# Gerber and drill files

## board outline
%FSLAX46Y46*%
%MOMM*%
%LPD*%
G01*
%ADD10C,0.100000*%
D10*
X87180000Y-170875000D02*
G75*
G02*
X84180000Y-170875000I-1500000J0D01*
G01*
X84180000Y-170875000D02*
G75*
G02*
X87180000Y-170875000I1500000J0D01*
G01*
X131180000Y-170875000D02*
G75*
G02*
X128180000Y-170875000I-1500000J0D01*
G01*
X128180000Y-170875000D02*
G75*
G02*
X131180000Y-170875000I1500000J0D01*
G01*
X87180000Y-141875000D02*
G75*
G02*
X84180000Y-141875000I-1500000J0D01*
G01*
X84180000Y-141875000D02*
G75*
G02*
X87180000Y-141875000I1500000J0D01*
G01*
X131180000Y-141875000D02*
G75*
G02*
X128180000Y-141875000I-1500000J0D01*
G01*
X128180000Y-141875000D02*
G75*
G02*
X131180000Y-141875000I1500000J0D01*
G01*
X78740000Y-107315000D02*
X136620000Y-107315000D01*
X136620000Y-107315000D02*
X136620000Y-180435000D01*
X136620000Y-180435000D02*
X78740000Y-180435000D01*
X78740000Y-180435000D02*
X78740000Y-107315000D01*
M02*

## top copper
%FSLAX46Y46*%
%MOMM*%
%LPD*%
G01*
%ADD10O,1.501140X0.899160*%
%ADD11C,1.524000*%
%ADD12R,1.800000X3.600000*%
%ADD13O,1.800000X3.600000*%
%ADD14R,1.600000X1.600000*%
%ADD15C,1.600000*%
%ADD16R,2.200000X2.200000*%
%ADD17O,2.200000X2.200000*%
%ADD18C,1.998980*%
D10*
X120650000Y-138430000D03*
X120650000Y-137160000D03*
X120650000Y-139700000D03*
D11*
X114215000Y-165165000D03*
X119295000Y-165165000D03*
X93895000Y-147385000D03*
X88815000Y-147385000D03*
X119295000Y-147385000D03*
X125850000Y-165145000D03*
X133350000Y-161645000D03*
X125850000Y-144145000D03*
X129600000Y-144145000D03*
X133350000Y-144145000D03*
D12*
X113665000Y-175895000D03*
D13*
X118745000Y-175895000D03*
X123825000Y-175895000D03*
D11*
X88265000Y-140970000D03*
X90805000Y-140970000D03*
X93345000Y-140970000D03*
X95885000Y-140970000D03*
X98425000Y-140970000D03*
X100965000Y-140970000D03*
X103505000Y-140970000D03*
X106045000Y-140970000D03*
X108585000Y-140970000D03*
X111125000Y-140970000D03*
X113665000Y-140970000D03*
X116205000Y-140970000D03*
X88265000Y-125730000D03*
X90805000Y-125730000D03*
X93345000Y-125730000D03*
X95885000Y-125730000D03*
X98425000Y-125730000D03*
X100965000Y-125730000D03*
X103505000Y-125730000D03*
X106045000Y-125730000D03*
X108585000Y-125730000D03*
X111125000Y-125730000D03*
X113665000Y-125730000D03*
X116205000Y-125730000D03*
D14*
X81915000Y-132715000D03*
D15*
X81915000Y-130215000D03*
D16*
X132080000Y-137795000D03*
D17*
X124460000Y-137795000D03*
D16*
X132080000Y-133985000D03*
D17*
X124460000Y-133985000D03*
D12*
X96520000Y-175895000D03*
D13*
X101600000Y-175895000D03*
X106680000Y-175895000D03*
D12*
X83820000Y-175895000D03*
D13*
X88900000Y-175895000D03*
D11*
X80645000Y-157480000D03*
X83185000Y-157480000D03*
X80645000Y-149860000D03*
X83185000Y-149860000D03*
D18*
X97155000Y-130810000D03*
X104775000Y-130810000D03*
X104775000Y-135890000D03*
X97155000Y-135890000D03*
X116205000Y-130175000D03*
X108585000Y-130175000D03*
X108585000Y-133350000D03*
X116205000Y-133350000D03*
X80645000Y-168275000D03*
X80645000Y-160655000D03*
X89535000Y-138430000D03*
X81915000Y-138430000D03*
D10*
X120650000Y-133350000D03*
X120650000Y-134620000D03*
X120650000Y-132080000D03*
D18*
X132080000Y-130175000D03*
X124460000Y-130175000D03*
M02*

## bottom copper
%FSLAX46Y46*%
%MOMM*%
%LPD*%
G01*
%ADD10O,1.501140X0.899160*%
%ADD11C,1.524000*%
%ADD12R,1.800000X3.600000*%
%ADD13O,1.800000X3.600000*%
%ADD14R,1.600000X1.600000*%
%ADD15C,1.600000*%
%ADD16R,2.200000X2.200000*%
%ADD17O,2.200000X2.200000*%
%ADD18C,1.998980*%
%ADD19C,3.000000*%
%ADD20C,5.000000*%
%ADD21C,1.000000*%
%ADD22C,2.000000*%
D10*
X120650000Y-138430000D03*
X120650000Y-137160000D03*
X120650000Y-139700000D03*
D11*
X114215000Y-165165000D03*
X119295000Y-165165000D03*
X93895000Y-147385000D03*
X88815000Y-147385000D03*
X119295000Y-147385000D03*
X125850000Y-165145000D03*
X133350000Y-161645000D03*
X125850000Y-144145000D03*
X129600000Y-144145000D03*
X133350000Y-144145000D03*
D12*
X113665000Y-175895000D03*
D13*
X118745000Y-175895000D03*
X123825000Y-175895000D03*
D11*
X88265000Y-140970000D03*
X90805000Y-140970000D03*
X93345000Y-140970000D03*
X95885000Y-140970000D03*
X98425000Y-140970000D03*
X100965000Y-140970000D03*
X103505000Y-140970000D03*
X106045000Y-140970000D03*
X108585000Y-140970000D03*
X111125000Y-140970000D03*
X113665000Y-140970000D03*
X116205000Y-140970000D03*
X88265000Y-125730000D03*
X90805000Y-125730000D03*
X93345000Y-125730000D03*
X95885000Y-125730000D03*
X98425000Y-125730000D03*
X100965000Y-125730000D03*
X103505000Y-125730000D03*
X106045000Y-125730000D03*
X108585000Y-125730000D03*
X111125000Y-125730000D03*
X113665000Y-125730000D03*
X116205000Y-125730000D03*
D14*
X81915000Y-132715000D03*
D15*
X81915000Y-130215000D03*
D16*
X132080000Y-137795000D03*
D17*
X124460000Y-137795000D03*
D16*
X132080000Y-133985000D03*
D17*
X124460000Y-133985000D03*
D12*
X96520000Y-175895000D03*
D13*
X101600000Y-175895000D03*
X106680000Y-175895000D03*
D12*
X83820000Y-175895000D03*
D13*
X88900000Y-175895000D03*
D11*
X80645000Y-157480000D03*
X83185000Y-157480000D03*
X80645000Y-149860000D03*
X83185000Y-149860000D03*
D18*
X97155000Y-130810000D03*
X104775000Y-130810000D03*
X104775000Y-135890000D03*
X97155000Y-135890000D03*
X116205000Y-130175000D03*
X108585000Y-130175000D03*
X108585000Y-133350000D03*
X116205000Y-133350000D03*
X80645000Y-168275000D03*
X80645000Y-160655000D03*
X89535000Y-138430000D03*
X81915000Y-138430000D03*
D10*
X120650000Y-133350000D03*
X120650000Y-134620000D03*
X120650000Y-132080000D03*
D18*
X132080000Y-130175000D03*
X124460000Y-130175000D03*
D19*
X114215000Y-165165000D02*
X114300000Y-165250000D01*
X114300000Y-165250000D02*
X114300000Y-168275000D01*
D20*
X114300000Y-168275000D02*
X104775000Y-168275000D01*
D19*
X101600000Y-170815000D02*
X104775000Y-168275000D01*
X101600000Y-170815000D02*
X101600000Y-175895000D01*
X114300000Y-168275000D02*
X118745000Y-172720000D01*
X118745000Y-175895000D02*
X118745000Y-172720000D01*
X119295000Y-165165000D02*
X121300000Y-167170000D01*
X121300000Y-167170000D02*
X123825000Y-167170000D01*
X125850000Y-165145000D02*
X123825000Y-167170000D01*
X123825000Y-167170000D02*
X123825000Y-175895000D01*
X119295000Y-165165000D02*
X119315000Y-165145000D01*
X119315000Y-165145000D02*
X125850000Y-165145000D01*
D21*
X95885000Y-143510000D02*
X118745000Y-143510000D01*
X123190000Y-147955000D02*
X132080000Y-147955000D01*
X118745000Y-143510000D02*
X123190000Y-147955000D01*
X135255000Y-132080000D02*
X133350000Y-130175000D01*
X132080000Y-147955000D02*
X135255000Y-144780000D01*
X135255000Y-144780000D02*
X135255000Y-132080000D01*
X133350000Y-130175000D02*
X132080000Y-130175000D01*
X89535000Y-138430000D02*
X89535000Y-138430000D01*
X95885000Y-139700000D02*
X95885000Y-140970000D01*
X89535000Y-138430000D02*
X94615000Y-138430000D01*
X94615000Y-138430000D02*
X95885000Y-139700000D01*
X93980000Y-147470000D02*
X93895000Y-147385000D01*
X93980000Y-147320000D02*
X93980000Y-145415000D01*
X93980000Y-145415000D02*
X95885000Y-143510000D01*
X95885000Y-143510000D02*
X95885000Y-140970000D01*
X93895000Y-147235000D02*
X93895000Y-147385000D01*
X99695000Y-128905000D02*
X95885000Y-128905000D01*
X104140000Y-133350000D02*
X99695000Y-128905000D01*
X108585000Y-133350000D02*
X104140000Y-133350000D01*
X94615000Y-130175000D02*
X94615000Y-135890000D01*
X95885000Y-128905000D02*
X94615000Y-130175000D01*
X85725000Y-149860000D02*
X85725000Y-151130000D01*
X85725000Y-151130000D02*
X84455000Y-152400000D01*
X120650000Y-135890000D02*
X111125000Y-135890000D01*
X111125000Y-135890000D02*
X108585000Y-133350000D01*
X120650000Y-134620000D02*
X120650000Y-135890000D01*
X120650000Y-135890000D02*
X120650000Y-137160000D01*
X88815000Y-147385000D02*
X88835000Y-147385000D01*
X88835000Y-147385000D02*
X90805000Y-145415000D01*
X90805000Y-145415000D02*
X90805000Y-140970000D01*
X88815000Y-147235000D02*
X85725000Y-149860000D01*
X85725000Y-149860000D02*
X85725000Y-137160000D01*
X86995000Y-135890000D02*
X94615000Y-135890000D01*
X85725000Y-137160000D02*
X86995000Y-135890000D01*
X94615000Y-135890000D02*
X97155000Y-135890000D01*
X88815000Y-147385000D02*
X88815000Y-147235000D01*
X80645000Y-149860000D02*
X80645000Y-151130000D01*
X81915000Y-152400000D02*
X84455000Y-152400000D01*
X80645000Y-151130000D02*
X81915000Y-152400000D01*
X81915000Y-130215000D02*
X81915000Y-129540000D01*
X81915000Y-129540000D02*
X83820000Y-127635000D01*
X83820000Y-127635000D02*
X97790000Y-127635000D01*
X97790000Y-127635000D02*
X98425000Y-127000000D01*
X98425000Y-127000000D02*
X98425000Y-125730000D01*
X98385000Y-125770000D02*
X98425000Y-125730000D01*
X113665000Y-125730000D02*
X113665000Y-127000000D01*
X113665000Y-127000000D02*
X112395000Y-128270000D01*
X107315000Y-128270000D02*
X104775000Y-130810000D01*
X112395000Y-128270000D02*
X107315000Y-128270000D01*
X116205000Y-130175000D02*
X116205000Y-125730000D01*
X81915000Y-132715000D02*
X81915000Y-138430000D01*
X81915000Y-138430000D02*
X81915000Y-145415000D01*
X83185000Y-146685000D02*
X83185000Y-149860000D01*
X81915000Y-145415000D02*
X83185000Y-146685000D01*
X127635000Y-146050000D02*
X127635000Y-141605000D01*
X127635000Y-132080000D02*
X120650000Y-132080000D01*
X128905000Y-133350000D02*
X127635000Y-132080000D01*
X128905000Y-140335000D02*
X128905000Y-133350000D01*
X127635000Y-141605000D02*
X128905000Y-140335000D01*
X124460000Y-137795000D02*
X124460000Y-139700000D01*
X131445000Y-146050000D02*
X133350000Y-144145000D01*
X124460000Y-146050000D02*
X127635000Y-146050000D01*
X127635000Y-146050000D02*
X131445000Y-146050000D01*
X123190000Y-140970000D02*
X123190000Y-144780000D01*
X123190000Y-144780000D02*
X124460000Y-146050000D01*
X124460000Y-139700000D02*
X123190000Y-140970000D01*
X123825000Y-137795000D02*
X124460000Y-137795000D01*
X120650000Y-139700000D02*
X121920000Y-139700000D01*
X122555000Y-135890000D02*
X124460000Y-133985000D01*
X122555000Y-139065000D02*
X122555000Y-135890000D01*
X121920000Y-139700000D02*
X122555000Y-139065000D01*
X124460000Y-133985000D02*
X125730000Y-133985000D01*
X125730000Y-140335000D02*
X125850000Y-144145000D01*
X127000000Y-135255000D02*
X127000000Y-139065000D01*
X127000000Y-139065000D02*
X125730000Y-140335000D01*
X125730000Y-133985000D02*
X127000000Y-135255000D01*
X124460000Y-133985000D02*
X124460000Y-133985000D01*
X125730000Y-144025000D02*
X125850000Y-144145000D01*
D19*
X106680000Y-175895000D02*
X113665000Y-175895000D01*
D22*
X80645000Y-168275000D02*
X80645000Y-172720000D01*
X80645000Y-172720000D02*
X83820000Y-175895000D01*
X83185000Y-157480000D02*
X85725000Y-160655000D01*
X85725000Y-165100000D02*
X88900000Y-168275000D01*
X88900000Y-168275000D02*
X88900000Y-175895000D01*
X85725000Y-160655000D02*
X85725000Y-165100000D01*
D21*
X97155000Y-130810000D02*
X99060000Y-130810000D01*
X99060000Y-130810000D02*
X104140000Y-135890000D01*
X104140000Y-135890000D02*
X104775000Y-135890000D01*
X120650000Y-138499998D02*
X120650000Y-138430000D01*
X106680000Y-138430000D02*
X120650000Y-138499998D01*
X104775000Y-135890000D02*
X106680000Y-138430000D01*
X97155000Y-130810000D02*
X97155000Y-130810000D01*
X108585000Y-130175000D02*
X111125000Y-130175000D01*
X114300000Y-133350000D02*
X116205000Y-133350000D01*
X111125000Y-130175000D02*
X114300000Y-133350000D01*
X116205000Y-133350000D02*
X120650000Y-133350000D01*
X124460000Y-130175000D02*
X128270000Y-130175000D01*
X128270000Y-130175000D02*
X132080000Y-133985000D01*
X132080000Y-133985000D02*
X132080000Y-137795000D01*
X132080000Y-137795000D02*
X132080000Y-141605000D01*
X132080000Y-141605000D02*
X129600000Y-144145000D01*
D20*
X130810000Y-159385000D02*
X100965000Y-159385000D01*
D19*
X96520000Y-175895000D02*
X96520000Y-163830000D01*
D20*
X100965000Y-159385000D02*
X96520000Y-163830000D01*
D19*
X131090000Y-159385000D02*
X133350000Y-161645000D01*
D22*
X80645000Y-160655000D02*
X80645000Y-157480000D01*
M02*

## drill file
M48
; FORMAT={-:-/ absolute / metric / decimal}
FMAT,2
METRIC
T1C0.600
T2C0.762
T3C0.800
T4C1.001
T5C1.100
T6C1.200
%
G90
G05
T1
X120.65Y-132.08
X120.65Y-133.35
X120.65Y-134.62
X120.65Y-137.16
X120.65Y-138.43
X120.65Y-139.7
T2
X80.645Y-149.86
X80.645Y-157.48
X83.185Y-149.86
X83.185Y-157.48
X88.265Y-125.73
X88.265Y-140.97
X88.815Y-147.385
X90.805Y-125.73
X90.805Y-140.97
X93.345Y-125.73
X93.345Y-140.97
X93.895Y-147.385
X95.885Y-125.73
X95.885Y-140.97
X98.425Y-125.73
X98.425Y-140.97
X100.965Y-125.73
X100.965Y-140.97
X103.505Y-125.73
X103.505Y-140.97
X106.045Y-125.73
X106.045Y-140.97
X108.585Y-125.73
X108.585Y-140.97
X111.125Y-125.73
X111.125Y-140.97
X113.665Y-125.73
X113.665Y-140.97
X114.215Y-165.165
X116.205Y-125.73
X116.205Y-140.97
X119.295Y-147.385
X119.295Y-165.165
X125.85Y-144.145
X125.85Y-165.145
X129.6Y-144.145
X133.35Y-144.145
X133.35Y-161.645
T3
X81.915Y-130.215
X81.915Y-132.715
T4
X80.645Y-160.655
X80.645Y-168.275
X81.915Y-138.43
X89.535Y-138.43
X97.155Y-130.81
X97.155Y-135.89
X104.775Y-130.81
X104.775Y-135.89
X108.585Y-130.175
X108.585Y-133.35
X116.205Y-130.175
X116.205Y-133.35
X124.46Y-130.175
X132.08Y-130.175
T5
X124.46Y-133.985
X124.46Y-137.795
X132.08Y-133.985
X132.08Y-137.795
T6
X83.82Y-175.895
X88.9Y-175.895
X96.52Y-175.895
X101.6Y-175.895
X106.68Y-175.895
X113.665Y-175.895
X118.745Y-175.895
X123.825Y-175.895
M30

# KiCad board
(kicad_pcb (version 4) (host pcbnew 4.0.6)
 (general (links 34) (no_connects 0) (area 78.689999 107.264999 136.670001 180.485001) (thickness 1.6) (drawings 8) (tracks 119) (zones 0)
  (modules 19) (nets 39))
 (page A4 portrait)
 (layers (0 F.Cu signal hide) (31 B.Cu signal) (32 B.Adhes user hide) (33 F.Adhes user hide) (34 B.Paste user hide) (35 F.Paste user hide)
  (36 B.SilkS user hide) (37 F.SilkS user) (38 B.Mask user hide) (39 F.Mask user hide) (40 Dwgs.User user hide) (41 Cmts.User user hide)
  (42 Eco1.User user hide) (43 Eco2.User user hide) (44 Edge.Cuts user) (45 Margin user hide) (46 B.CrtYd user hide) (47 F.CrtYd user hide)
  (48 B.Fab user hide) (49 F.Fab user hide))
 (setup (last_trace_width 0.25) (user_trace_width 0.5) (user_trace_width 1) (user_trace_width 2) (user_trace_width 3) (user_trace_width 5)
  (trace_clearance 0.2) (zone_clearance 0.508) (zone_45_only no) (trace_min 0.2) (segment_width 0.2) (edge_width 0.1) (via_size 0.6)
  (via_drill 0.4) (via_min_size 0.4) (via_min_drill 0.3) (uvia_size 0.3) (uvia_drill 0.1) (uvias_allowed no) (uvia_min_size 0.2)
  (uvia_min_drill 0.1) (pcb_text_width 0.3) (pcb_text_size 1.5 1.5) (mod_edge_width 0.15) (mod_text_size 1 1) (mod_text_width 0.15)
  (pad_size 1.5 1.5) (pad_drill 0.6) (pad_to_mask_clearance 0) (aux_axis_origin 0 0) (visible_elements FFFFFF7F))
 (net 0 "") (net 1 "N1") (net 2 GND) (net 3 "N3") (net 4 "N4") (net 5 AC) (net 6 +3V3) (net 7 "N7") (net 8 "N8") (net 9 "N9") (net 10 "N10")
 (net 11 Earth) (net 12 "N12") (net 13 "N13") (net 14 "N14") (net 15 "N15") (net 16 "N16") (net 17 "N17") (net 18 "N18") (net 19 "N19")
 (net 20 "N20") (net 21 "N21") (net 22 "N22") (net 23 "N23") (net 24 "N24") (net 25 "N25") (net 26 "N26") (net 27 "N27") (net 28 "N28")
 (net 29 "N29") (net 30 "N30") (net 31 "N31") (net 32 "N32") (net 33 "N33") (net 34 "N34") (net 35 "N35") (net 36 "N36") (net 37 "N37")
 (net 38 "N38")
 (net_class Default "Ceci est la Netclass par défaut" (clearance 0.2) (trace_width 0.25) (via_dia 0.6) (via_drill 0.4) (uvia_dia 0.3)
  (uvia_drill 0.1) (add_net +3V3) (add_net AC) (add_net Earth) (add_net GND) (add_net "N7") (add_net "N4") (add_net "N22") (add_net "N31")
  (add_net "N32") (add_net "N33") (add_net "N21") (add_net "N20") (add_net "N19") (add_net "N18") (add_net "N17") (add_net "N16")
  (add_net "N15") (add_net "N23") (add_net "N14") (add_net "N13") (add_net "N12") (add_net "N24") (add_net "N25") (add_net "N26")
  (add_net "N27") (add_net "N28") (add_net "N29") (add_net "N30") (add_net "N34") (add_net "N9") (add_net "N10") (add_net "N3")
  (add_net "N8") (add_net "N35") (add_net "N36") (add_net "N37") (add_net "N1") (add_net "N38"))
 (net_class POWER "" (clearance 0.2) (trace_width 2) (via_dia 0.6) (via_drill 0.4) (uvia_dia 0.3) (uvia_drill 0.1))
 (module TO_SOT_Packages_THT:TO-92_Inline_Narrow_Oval (layer F.Cu) (at 120.65 139.7 90)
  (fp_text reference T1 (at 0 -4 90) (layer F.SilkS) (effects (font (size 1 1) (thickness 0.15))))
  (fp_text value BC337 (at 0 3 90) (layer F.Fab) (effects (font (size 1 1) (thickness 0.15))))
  (pad 2 thru_hole oval (at 1.27 0 270) (size 0.89916 1.50114) (drill 0.6) (layers *.Cu *.Mask) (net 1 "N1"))
  (pad 3 thru_hole oval (at 2.54 0 270) (size 0.89916 1.50114) (drill 0.6) (layers *.Cu *.Mask) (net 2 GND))
  (pad 1 thru_hole oval (at 0 0 270) (size 0.89916 1.50114) (drill 0.6) (layers *.Cu *.Mask) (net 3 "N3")))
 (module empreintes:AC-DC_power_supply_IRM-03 (layer F.Cu) (at 122.555 168.275 180)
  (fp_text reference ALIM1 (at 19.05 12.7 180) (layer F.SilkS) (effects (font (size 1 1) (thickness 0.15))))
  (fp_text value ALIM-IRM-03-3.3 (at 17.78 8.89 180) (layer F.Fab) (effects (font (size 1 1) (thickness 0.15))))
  (pad 3 thru_hole circle (at 8.34 3.11 180) (size 1.524 1.524) (drill 0.762) (layers *.Cu *.Mask) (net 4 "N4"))
  (pad 1 thru_hole circle (at 3.26 3.11 180) (size 1.524 1.524) (drill 0.762) (layers *.Cu *.Mask) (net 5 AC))
  (pad 16 thru_hole circle (at 28.66 20.89 180) (size 1.524 1.524) (drill 0.762) (layers *.Cu *.Mask) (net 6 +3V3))
  (pad 14 thru_hole circle (at 33.74 20.89 180) (size 1.524 1.524) (drill 0.762) (layers *.Cu *.Mask) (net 2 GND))
  (pad 13 thru_hole circle (at 3.26 20.89 180) (size 1.524 1.524) (drill 0.762) (layers *.Cu *.Mask) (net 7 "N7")))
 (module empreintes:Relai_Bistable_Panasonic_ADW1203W (layer F.Cu) (at 133.35 144.145)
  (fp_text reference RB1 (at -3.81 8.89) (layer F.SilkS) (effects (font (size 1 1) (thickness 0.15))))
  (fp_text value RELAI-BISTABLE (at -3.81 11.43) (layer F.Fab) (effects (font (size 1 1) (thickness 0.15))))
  (pad 3 thru_hole circle (at -7.5 21) (size 1.524 1.524) (drill 0.762) (layers *.Cu *.Mask) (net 5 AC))
  (pad 5 thru_hole circle (at 0 17.5) (size 1.524 1.524) (drill 0.762) (layers *.Cu *.Mask) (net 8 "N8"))
  (pad -1 thru_hole circle (at -7.5 0) (size 1.524 1.524) (drill 0.762) (layers *.Cu *.Mask) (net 3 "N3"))
  (pad +7 thru_hole circle (at -3.75 0) (size 1.524 1.524) (drill 0.762) (layers *.Cu *.Mask) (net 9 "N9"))
  (pad -6 thru_hole circle (at 0 0) (size 1.524 1.524) (drill 0.762) (layers *.Cu *.Mask) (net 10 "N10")))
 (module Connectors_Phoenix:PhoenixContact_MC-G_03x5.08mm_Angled (layer F.Cu) (at 113.665 175.895)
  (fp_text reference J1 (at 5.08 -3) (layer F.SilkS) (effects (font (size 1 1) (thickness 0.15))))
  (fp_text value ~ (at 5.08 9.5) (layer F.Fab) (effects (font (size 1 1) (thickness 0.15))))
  (pad 1 thru_hole rect (at 0 0) (size 1.8 3.6) (drill 1.2) (layers *.Cu *.Mask) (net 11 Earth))
  (pad 2 thru_hole oval (at 5.08 0) (size 1.8 3.6) (drill 1.2) (layers *.Cu *.Mask) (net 4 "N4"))
  (pad 3 thru_hole oval (at 10.16 0) (size 1.8 3.6) (drill 1.2) (layers *.Cu *.Mask) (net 5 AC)))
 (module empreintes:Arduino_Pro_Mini (layer F.Cu) (at 116.205 133.35 90)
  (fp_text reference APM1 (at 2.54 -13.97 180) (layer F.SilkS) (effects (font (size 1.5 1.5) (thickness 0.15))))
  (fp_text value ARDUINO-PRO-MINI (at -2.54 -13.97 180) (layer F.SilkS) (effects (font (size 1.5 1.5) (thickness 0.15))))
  (pad 24 thru_hole circle (at -7.62 -27.94 90) (size 1.524 1.524) (drill 0.762) (layers *.Cu *.Mask F.SilkS) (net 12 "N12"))
  (pad 23 thru_hole circle (at -7.62 -25.4 90) (size 1.524 1.524) (drill 0.762) (layers *.Cu *.Mask F.SilkS) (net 2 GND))
  (pad 22 thru_hole circle (at -7.62 -22.86 90) (size 1.524 1.524) (drill 0.762) (layers *.Cu *.Mask F.SilkS) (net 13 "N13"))
  (pad 21 thru_hole circle (at -7.62 -20.32 90) (size 1.524 1.524) (drill 0.762) (layers *.Cu *.Mask F.SilkS) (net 6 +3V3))
  (pad 20 thru_hole circle (at -7.62 -17.78 90) (size 1.524 1.524) (drill 0.762) (layers *.Cu *.Mask F.SilkS) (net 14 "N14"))
  (pad 19 thru_hole circle (at -7.62 -15.24 90) (size 1.524 1.524) (drill 0.762) (layers *.Cu *.Mask F.SilkS) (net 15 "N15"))
  (pad 18 thru_hole circle (at -7.62 -12.7 90) (size 1.524 1.524) (drill 0.762) (layers *.Cu *.Mask F.SilkS) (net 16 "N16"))
  (pad 17 thru_hole circle (at -7.62 -10.16 90) (size 1.524 1.524) (drill 0.762) (layers *.Cu *.Mask F.SilkS) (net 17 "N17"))
  (pad 16 thru_hole circle (at -7.62 -7.62 90) (size 1.524 1.524) (drill 0.762) (layers *.Cu *.Mask F.SilkS) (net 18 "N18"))
  (pad 15 thru_hole circle (at -7.62 -5.08 90) (size 1.524 1.524) (drill 0.762) (layers *.Cu *.Mask F.SilkS) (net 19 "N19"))
  (pad 14 thru_hole circle (at -7.62 -2.54 90) (size 1.524 1.524) (drill 0.762) (layers *.Cu *.Mask F.SilkS) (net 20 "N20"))
  (pad 13 thru_hole circle (at -7.62 0 90) (size 1.524 1.524) (drill 0.762) (layers *.Cu *.Mask F.SilkS) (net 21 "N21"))
  (pad 1 thru_hole circle (at 7.62 -27.94 90) (size 1.524 1.524) (drill 0.762) (layers *.Cu *.Mask F.SilkS) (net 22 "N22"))
  (pad 2 thru_hole circle (at 7.62 -25.4 90) (size 1.524 1.524) (drill 0.762) (layers *.Cu *.Mask F.SilkS) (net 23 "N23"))
  (pad 3 thru_hole circle (at 7.62 -22.86 90) (size 1.524 1.524) (drill 0.762) (layers *.Cu *.Mask F.SilkS) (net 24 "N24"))
  (pad 4 thru_hole circle (at 7.62 -20.32 90) (size 1.524 1.524) (drill 0.762) (layers *.Cu *.Mask F.SilkS) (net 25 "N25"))
  (pad 5 thru_hole circle (at 7.62 -17.78 90) (size 1.524 1.524) (drill 0.762) (layers *.Cu *.Mask F.SilkS) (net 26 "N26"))
  (pad 6 thru_hole circle (at 7.62 -15.24 90) (size 1.524 1.524) (drill 0.762) (layers *.Cu *.Mask F.SilkS) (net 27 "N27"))
  (pad 7 thru_hole circle (at 7.62 -12.7 90) (size 1.524 1.524) (drill 0.762) (layers *.Cu *.Mask F.SilkS) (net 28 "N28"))
  (pad 8 thru_hole circle (at 7.62 -10.16 90) (size 1.524 1.524) (drill 0.762) (layers *.Cu *.Mask F.SilkS) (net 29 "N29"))
  (pad 9 thru_hole circle (at 7.62 -7.62 90) (size 1.524 1.524) (drill 0.762) (layers *.Cu *.Mask F.SilkS) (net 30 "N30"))
  (pad 10 thru_hole circle (at 7.62 -5.08 90) (size 1.524 1.524) (drill 0.762) (layers *.Cu *.Mask F.SilkS) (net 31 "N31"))
  (pad 11 thru_hole circle (at 7.62 -2.54 90) (size 1.524 1.524) (drill 0.762) (layers *.Cu *.Mask F.SilkS) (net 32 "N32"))
  (pad 12 thru_hole circle (at 7.62 0 90) (size 1.524 1.524) (drill 0.762) (layers *.Cu *.Mask F.SilkS) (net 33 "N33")))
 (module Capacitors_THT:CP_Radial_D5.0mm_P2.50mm (layer F.Cu) (at 81.915 132.715 90)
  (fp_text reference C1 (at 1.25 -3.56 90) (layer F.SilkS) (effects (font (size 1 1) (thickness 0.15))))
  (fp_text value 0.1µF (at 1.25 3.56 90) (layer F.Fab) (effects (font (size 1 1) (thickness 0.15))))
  (pad 1 thru_hole rect (at 0 0 90) (size 1.6 1.6) (drill 0.8) (layers *.Cu *.Mask) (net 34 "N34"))
  (pad 2 thru_hole circle (at 2.5 0 90) (size 1.6 1.6) (drill 0.8) (layers *.Cu *.Mask) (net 26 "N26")))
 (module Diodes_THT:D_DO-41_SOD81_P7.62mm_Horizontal (layer F.Cu) (at 132.08 137.795 180)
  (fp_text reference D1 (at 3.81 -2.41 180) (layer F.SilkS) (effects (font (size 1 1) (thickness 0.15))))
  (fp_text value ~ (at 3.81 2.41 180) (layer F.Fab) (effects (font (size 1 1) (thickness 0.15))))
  (pad 1 thru_hole rect (at 0 0 180) (size 2.2 2.2) (drill 1.1) (layers *.Cu *.Mask) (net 9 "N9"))
  (pad 2 thru_hole oval (at 7.62 0 180) (size 2.2 2.2) (drill 1.1) (layers *.Cu *.Mask) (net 10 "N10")))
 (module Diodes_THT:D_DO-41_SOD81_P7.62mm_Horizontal (layer F.Cu) (at 132.08 133.985 180)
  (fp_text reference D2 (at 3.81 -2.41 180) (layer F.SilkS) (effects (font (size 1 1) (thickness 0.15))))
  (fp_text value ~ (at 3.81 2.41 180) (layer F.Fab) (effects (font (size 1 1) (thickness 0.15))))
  (pad 1 thru_hole rect (at 0 0 180) (size 2.2 2.2) (drill 1.1) (layers *.Cu *.Mask) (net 9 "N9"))
  (pad 2 thru_hole oval (at 7.62 0 180) (size 2.2 2.2) (drill 1.1) (layers *.Cu *.Mask) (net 3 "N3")))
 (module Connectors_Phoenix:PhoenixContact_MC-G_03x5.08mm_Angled (layer F.Cu) (at 96.52 175.895)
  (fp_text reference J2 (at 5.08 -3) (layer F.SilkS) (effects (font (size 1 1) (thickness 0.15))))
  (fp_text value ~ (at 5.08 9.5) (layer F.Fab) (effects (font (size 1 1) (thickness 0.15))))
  (pad 1 thru_hole rect (at 0 0) (size 1.8 3.6) (drill 1.2) (layers *.Cu *.Mask) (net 8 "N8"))
  (pad 2 thru_hole oval (at 5.08 0) (size 1.8 3.6) (drill 1.2) (layers *.Cu *.Mask) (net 4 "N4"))
  (pad 3 thru_hole oval (at 10.16 0) (size 1.8 3.6) (drill 1.2) (layers *.Cu *.Mask) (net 11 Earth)))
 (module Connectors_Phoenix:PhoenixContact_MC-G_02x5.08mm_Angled (layer F.Cu) (at 83.82 175.895)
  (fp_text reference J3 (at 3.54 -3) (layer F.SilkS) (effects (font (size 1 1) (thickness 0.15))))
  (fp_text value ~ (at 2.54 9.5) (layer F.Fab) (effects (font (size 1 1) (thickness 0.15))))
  (pad 1 thru_hole rect (at 0 0) (size 1.8 3.6) (drill 1.2) (layers *.Cu *.Mask) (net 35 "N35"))
  (pad 2 thru_hole oval (at 5.08 0) (size 1.8 3.6) (drill 1.2) (layers *.Cu *.Mask) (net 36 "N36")))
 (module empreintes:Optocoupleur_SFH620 (layer F.Cu) (at 83.185 153.67 270)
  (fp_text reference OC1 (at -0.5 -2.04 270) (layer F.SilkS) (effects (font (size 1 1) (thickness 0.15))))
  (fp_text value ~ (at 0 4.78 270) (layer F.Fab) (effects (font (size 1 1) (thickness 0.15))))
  (pad 2 thru_hole circle (at 3.81 2.54 270) (size 1.524 1.524) (drill 0.762) (layers *.Cu *.Mask) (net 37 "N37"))
  (pad 1 thru_hole circle (at 3.81 0 270) (size 1.524 1.524) (drill 0.762) (layers *.Cu *.Mask) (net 36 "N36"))
  (pad 3 thru_hole circle (at -3.81 2.54 270) (size 1.524 1.524) (drill 0.762) (layers *.Cu *.Mask) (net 2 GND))
  (pad 4 thru_hole circle (at -3.81 0 270) (size 1.524 1.524) (drill 0.762) (layers *.Cu *.Mask) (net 34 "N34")))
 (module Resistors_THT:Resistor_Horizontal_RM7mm (layer F.Cu) (at 97.155 130.81)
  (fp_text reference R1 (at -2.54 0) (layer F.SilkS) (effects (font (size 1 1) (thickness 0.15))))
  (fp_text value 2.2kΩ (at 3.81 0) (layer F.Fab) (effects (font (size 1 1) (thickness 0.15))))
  (pad 1 thru_hole circle (at 0 0) (size 1.99898 1.99898) (drill 1.00076) (layers *.Cu *.SilkS *.Mask) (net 1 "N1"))
  (pad 2 thru_hole circle (at 7.62 0) (size 1.99898 1.99898) (drill 1.00076) (layers *.Cu *.SilkS *.Mask) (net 32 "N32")))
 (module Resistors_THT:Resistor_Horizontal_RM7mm (layer F.Cu) (at 104.775 135.89 180)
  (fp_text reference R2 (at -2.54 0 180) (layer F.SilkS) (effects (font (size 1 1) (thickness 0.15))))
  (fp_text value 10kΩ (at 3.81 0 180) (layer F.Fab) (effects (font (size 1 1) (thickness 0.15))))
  (pad 1 thru_hole circle (at 0 0 180) (size 1.99898 1.99898) (drill 1.00076) (layers *.Cu *.SilkS *.Mask) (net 1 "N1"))
  (pad 2 thru_hole circle (at 7.62 0 180) (size 1.99898 1.99898) (drill 1.00076) (layers *.Cu *.SilkS *.Mask) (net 2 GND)))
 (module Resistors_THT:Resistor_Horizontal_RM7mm (layer F.Cu) (at 116.205 130.175 180)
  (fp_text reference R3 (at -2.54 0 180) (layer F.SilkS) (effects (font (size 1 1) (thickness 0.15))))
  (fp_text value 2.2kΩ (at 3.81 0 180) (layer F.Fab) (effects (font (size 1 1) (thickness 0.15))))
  (pad 1 thru_hole circle (at 0 0 180) (size 1.99898 1.99898) (drill 1.00076) (layers *.Cu *.SilkS *.Mask) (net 33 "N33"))
  (pad 2 thru_hole circle (at 7.62 0 180) (size 1.99898 1.99898) (drill 1.00076) (layers *.Cu *.SilkS *.Mask) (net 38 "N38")))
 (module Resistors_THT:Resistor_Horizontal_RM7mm (layer F.Cu) (at 108.585 133.35)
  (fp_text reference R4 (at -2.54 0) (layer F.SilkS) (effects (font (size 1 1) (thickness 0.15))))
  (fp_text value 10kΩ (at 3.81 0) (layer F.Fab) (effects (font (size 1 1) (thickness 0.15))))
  (pad 1 thru_hole circle (at 0 0) (size 1.99898 1.99898) (drill 1.00076) (layers *.Cu *.SilkS *.Mask) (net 2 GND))
  (pad 2 thru_hole circle (at 7.62 0) (size 1.99898 1.99898) (drill 1.00076) (layers *.Cu *.SilkS *.Mask) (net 38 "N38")))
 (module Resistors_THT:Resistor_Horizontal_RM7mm (layer F.Cu) (at 80.645 168.275 90)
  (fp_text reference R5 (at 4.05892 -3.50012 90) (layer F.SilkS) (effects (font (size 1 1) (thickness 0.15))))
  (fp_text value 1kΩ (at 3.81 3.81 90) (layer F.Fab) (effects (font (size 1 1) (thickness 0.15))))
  (pad 1 thru_hole circle (at 0 0 90) (size 1.99898 1.99898) (drill 1.00076) (layers *.Cu *.SilkS *.Mask) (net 35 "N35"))
  (pad 2 thru_hole circle (at 7.62 0 90) (size 1.99898 1.99898) (drill 1.00076) (layers *.Cu *.SilkS *.Mask) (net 37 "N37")))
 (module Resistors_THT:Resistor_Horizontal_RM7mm (layer F.Cu) (at 89.535 138.43 180)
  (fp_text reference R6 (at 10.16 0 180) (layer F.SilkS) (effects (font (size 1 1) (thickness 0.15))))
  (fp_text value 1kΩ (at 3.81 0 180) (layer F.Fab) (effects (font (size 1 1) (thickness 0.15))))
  (pad 1 thru_hole circle (at 0 0 180) (size 1.99898 1.99898) (drill 1.00076) (layers *.Cu *.SilkS *.Mask) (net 6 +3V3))
  (pad 2 thru_hole circle (at 7.62 0 180) (size 1.99898 1.99898) (drill 1.00076) (layers *.Cu *.SilkS *.Mask) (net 34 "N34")))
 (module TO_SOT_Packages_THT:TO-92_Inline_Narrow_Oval (layer F.Cu) (at 120.65 132.08 270)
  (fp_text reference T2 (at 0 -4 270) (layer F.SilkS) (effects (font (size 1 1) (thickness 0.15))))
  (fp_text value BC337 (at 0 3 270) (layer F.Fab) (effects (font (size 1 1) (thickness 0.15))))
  (pad 2 thru_hole oval (at 1.27 0 90) (size 0.89916 1.50114) (drill 0.6) (layers *.Cu *.Mask) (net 38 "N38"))
  (pad 3 thru_hole oval (at 2.54 0 90) (size 0.89916 1.50114) (drill 0.6) (layers *.Cu *.Mask) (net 2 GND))
  (pad 1 thru_hole oval (at 0 0 90) (size 0.89916 1.50114) (drill 0.6) (layers *.Cu *.Mask) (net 10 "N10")))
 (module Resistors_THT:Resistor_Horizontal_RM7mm (layer F.Cu) (at 132.08 130.175 180)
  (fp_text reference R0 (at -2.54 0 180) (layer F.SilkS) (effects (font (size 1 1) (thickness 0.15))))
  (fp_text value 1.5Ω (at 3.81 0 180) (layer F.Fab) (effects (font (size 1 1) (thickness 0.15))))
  (pad 1 thru_hole circle (at 0 0 180) (size 1.99898 1.99898) (drill 1.00076) (layers *.Cu *.SilkS *.Mask) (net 6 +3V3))
  (pad 2 thru_hole circle (at 7.62 0 180) (size 1.99898 1.99898) (drill 1.00076) (layers *.Cu *.SilkS *.Mask) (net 9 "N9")))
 (gr_circle (center 85.68 170.875) (end 85.68 172.375) (layer Edge.Cuts) (width 0.1))
 (gr_circle (center 129.68 170.875) (end 129.68 172.375) (layer Edge.Cuts) (width 0.1))
 (gr_circle (center 85.68 141.875) (end 85.68 143.375) (layer Edge.Cuts) (width 0.1))
 (gr_circle (center 129.68 141.875) (end 129.68 143.375) (layer Edge.Cuts) (width 0.1))
 (gr_line (start 78.74 107.315) (end 136.62 107.315) (angle 90) (layer Edge.Cuts) (width 0.1))
 (gr_line (start 136.62 107.315) (end 136.62 180.435) (angle 90) (layer Edge.Cuts) (width 0.1))
 (gr_line (start 136.62 180.435) (end 78.74 180.435) (angle 90) (layer Edge.Cuts) (width 0.1))
 (gr_line (start 78.74 180.435) (end 78.74 107.315) (angle 90) (layer Edge.Cuts) (width 0.1))
 (segment (start 114.215 165.165) (end 114.3 165.25) (width 3) (layer B.Cu) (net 4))
 (segment (start 114.3 165.25) (end 114.3 168.275) (width 3) (layer B.Cu) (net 4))
 (segment (start 114.3 168.275) (end 104.775 168.275) (width 5) (layer B.Cu) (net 4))
 (segment (start 101.6 170.815) (end 104.775 168.275) (width 3) (layer B.Cu) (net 4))
 (segment (start 101.6 170.815) (end 101.6 175.895) (width 3) (layer B.Cu) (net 4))
 (segment (start 114.3 168.275) (end 118.745 172.72) (width 3) (layer B.Cu) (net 4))
 (segment (start 118.745 175.895) (end 118.745 172.72) (width 3) (layer B.Cu) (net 4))
 (segment (start 119.295 165.165) (end 121.3 167.17) (width 3) (layer B.Cu) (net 5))
 (segment (start 121.3 167.17) (end 123.825 167.17) (width 3) (layer B.Cu) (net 5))
 (segment (start 125.85 165.145) (end 123.825 167.17) (width 3) (layer B.Cu) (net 5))
 (segment (start 123.825 167.17) (end 123.825 175.895) (width 3) (layer B.Cu) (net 5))
 (segment (start 119.295 165.165) (end 119.315 165.145) (width 3) (layer B.Cu) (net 5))
 (segment (start 119.315 165.145) (end 125.85 165.145) (width 3) (layer B.Cu) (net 5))
 (segment (start 95.885 143.51) (end 118.745 143.51) (width 1) (layer B.Cu) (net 6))
 (segment (start 123.19 147.955) (end 132.08 147.955) (width 1) (layer B.Cu) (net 6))
 (segment (start 118.745 143.51) (end 123.19 147.955) (width 1) (layer B.Cu) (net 6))
 (segment (start 135.255 132.08) (end 133.35 130.175) (width 1) (layer B.Cu) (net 6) (status 20))
 (segment (start 132.08 147.955) (end 135.255 144.78) (width 1) (layer B.Cu) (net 6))
 (segment (start 135.255 144.78) (end 135.255 132.08) (width 1) (layer B.Cu) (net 6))
 (segment (start 133.35 130.175) (end 132.08 130.175) (width 1) (layer B.Cu) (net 6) (status 20))
 (segment (start 89.535 138.43) (end 89.535 138.43) (width 1) (layer B.Cu) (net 6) (status 30))
 (segment (start 95.885 139.7) (end 95.885 140.97) (width 1) (layer B.Cu) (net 6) (status 20))
 (segment (start 89.535 138.43) (end 94.615 138.43) (width 1) (layer B.Cu) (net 6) (status 10))
 (segment (start 94.615 138.43) (end 95.885 139.7) (width 1) (layer B.Cu) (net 6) (status 10))
 (segment (start 93.98 147.47) (end 93.895 147.385) (width 1) (layer B.Cu) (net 6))
 (segment (start 93.98 147.32) (end 93.98 145.415) (width 1) (layer B.Cu) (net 6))
 (segment (start 93.98 145.415) (end 95.885 143.51) (width 1) (layer B.Cu) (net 6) (status 20))
 (segment (start 95.885 143.51) (end 95.885 140.97) (width 1) (layer B.Cu) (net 6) (status 20))
 (segment (start 93.895 147.235) (end 93.895 147.385) (width 1) (layer B.Cu) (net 6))
 (segment (start 99.695 128.905) (end 95.885 128.905) (width 1) (layer B.Cu) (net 2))
 (segment (start 104.14 133.35) (end 99.695 128.905) (width 1) (layer B.Cu) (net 2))
 (segment (start 108.585 133.35) (end 104.14 133.35) (width 1) (layer B.Cu) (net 2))
 (segment (start 94.615 130.175) (end 94.615 135.89) (width 1) (layer B.Cu) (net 2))
 (segment (start 95.885 128.905) (end 94.615 130.175) (width 1) (layer B.Cu) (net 2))
 (segment (start 85.725 149.86) (end 85.725 151.13) (width 1) (layer B.Cu) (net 2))
 (segment (start 85.725 151.13) (end 84.455 152.4) (width 1) (layer B.Cu) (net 2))
 (segment (start 120.65 135.89) (end 111.125 135.89) (width 1) (layer B.Cu) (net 2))
 (segment (start 111.125 135.89) (end 108.585 133.35) (width 1) (layer B.Cu) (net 2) (status 20))
 (segment (start 120.65 134.62) (end 120.65 135.89) (width 1) (layer B.Cu) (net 2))
 (segment (start 120.65 135.89) (end 120.65 137.16) (width 1) (layer B.Cu) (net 2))
 (segment (start 88.815 147.385) (end 88.835 147.385) (width 1) (layer B.Cu) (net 2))
 (segment (start 88.835 147.385) (end 90.805 145.415) (width 1) (layer B.Cu) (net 2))
 (segment (start 90.805 145.415) (end 90.805 140.97) (width 1) (layer B.Cu) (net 2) (status 20))
 (segment (start 88.815 147.235) (end 85.725 149.86) (width 1) (layer B.Cu) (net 2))
 (segment (start 85.725 149.86) (end 85.725 137.16) (width 1) (layer B.Cu) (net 2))
 (segment (start 86.995 135.89) (end 94.615 135.89) (width 1) (layer B.Cu) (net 2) (status 20))
 (segment (start 85.725 137.16) (end 86.995 135.89) (width 1) (layer B.Cu) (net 2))
 (segment (start 94.615 135.89) (end 97.155 135.89) (width 1) (layer B.Cu) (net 2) (status 20))
 (segment (start 88.815 147.385) (end 88.815 147.235) (width 1) (layer B.Cu) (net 2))
 (segment (start 80.645 149.86) (end 80.645 151.13) (width 1) (layer B.Cu) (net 2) (status 30))
 (segment (start 81.915 152.4) (end 84.455 152.4) (width 1) (layer B.Cu) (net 2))
 (segment (start 80.645 151.13) (end 81.915 152.4) (width 1) (layer B.Cu) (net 2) (status 10))
 (segment (start 81.915 130.215) (end 81.915 129.54) (width 1) (layer B.Cu) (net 26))
 (segment (start 81.915 129.54) (end 83.82 127.635) (width 1) (layer B.Cu) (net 26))
 (segment (start 83.82 127.635) (end 97.79 127.635) (width 1) (layer B.Cu) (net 26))
 (segment (start 97.79 127.635) (end 98.425 127) (width 1) (layer B.Cu) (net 26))
 (segment (start 98.425 127) (end 98.425 125.73) (width 1) (layer B.Cu) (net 26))
 (segment (start 98.385 125.77) (end 98.425 125.73) (width 1) (layer B.Cu) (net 26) (status 30))
 (segment (start 113.665 125.73) (end 113.665 127) (width 1) (layer B.Cu) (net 32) (status 10))
 (segment (start 113.665 127) (end 112.395 128.27) (width 1) (layer B.Cu) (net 32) (status 10))
 (segment (start 107.315 128.27) (end 104.775 130.81) (width 1) (layer B.Cu) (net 32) (status 20))
 (segment (start 112.395 128.27) (end 107.315 128.27) (width 1) (layer B.Cu) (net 32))
 (segment (start 116.205 130.175) (end 116.205 125.73) (width 1) (layer B.Cu) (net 33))
 (segment (start 81.915 132.715) (end 81.915 138.43) (width 1) (layer B.Cu) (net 34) (status 10))
 (segment (start 81.915 138.43) (end 81.915 145.415) (width 1) (layer B.Cu) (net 34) (status 10))
 (segment (start 83.185 146.685) (end 83.185 149.86) (width 1) (layer B.Cu) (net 34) (status 30))
 (segment (start 81.915 145.415) (end 83.185 146.685) (width 1) (layer B.Cu) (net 34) (status 20))
 (segment (start 127.635 146.05) (end 127.635 141.605) (width 1) (layer B.Cu) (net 10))
 (segment (start 127.635 132.08) (end 120.65 132.08) (width 1) (layer B.Cu) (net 10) (status 20))
 (segment (start 128.905 133.35) (end 127.635 132.08) (width 1) (layer B.Cu) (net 10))
 (segment (start 128.905 140.335) (end 128.905 133.35) (width 1) (layer B.Cu) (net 10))
 (segment (start 127.635 141.605) (end 128.905 140.335) (width 1) (layer B.Cu) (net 10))
 (segment (start 124.46 137.795) (end 124.46 139.7) (width 1) (layer B.Cu) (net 10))
 (segment (start 131.445 146.05) (end 133.35 144.145) (width 1) (layer B.Cu) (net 10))
 (segment (start 124.46 146.05) (end 127.635 146.05) (width 1) (layer B.Cu) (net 10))
 (segment (start 127.635 146.05) (end 131.445 146.05) (width 1) (layer B.Cu) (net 10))
 (segment (start 123.19 140.97) (end 123.19 144.78) (width 1) (layer B.Cu) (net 10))
 (segment (start 123.19 144.78) (end 124.46 146.05) (width 1) (layer B.Cu) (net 10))
 (segment (start 124.46 139.7) (end 123.19 140.97) (width 1) (layer B.Cu) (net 10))
 (segment (start 123.825 137.795) (end 124.46 137.795) (width 1) (layer B.Cu) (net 10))
 (segment (start 120.65 139.7) (end 121.92 139.7) (width 1) (layer B.Cu) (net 3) (status 10))
 (segment (start 122.555 135.89) (end 124.46 133.985) (width 1) (layer B.Cu) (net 3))
 (segment (start 122.555 139.065) (end 122.555 135.89) (width 1) (layer B.Cu) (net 3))
 (segment (start 121.92 139.7) (end 122.555 139.065) (width 1) (layer B.Cu) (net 3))
 (segment (start 124.46 133.985) (end 125.73 133.985) (width 1) (layer B.Cu) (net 3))
 (segment (start 125.73 140.335) (end 125.85 144.145) (width 1) (layer B.Cu) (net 3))
 (segment (start 127 135.255) (end 127 139.065) (width 1) (layer B.Cu) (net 3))
 (segment (start 127 139.065) (end 125.73 140.335) (width 1) (layer B.Cu) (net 3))
 (segment (start 125.73 133.985) (end 127 135.255) (width 1) (layer B.Cu) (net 3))
 (segment (start 124.46 133.985) (end 124.46 133.985) (width 1) (layer B.Cu) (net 3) (status 10))
 (segment (start 125.73 144.025) (end 125.85 144.145) (width 1) (layer B.Cu) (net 3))
 (segment (start 106.68 175.895) (end 113.665 175.895) (width 3) (layer B.Cu) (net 11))
 (segment (start 80.645 168.275) (end 80.645 172.72) (width 2) (layer B.Cu) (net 35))
 (segment (start 80.645 172.72) (end 83.82 175.895) (width 2) (layer B.Cu) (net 35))
 (segment (start 83.185 157.48) (end 85.725 160.655) (width 2) (layer B.Cu) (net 36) (status 10))
 (segment (start 85.725 165.1) (end 88.9 168.275) (width 2) (layer B.Cu) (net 36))
 (segment (start 88.9 168.275) (end 88.9 175.895) (width 2) (layer B.Cu) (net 36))
 (segment (start 85.725 160.655) (end 85.725 165.1) (width 2) (layer B.Cu) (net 36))
 (segment (start 97.155 130.81) (end 99.06 130.81) (width 1) (layer B.Cu) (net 1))
 (segment (start 99.06 130.81) (end 104.14 135.89) (width 1) (layer B.Cu) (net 1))
 (segment (start 104.14 135.89) (end 104.775 135.89) (width 1) (layer B.Cu) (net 1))
 (segment (start 120.65 138.499998) (end 120.65 138.43) (width 1) (layer B.Cu) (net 1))
 (segment (start 106.68 138.43) (end 120.65 138.499998) (width 1) (layer B.Cu) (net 1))
 (segment (start 104.775 135.89) (end 106.68 138.43) (width 1) (layer B.Cu) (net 1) (status 10))
 (segment (start 97.155 130.81) (end 97.155 130.81) (width 1) (layer B.Cu) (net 1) (status 30))
 (segment (start 108.585 130.175) (end 111.125 130.175) (width 1) (layer B.Cu) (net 38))
 (segment (start 114.3 133.35) (end 116.205 133.35) (width 1) (layer B.Cu) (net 38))
 (segment (start 111.125 130.175) (end 114.3 133.35) (width 1) (layer B.Cu) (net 38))
 (segment (start 116.205 133.35) (end 120.65 133.35) (width 1) (layer B.Cu) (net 38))
 (segment (start 124.46 130.175) (end 128.27 130.175) (width 1) (layer B.Cu) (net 9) (status 10))
 (segment (start 128.27 130.175) (end 132.08 133.985) (width 1) (layer B.Cu) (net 9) (status 10))
 (segment (start 132.08 133.985) (end 132.08 137.795) (width 1) (layer B.Cu) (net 9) (status 10))
 (segment (start 132.08 137.795) (end 132.08 141.605) (width 1) (layer B.Cu) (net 9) (status 10))
 (segment (start 132.08 141.605) (end 129.6 144.145) (width 1) (layer B.Cu) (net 9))
 (segment (start 130.81 159.385) (end 100.965 159.385) (width 5) (layer B.Cu) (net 8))
 (segment (start 96.52 175.895) (end 96.52 163.83) (width 3) (layer B.Cu) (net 8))
 (segment (start 100.965 159.385) (end 96.52 163.83) (width 5) (layer B.Cu) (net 8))
 (segment (start 131.09 159.385) (end 133.35 161.645) (width 3) (layer B.Cu) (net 8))
 (segment (start 80.645 160.655) (end 80.645 157.48) (width 2) (layer B.Cu) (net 37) (status 10)))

